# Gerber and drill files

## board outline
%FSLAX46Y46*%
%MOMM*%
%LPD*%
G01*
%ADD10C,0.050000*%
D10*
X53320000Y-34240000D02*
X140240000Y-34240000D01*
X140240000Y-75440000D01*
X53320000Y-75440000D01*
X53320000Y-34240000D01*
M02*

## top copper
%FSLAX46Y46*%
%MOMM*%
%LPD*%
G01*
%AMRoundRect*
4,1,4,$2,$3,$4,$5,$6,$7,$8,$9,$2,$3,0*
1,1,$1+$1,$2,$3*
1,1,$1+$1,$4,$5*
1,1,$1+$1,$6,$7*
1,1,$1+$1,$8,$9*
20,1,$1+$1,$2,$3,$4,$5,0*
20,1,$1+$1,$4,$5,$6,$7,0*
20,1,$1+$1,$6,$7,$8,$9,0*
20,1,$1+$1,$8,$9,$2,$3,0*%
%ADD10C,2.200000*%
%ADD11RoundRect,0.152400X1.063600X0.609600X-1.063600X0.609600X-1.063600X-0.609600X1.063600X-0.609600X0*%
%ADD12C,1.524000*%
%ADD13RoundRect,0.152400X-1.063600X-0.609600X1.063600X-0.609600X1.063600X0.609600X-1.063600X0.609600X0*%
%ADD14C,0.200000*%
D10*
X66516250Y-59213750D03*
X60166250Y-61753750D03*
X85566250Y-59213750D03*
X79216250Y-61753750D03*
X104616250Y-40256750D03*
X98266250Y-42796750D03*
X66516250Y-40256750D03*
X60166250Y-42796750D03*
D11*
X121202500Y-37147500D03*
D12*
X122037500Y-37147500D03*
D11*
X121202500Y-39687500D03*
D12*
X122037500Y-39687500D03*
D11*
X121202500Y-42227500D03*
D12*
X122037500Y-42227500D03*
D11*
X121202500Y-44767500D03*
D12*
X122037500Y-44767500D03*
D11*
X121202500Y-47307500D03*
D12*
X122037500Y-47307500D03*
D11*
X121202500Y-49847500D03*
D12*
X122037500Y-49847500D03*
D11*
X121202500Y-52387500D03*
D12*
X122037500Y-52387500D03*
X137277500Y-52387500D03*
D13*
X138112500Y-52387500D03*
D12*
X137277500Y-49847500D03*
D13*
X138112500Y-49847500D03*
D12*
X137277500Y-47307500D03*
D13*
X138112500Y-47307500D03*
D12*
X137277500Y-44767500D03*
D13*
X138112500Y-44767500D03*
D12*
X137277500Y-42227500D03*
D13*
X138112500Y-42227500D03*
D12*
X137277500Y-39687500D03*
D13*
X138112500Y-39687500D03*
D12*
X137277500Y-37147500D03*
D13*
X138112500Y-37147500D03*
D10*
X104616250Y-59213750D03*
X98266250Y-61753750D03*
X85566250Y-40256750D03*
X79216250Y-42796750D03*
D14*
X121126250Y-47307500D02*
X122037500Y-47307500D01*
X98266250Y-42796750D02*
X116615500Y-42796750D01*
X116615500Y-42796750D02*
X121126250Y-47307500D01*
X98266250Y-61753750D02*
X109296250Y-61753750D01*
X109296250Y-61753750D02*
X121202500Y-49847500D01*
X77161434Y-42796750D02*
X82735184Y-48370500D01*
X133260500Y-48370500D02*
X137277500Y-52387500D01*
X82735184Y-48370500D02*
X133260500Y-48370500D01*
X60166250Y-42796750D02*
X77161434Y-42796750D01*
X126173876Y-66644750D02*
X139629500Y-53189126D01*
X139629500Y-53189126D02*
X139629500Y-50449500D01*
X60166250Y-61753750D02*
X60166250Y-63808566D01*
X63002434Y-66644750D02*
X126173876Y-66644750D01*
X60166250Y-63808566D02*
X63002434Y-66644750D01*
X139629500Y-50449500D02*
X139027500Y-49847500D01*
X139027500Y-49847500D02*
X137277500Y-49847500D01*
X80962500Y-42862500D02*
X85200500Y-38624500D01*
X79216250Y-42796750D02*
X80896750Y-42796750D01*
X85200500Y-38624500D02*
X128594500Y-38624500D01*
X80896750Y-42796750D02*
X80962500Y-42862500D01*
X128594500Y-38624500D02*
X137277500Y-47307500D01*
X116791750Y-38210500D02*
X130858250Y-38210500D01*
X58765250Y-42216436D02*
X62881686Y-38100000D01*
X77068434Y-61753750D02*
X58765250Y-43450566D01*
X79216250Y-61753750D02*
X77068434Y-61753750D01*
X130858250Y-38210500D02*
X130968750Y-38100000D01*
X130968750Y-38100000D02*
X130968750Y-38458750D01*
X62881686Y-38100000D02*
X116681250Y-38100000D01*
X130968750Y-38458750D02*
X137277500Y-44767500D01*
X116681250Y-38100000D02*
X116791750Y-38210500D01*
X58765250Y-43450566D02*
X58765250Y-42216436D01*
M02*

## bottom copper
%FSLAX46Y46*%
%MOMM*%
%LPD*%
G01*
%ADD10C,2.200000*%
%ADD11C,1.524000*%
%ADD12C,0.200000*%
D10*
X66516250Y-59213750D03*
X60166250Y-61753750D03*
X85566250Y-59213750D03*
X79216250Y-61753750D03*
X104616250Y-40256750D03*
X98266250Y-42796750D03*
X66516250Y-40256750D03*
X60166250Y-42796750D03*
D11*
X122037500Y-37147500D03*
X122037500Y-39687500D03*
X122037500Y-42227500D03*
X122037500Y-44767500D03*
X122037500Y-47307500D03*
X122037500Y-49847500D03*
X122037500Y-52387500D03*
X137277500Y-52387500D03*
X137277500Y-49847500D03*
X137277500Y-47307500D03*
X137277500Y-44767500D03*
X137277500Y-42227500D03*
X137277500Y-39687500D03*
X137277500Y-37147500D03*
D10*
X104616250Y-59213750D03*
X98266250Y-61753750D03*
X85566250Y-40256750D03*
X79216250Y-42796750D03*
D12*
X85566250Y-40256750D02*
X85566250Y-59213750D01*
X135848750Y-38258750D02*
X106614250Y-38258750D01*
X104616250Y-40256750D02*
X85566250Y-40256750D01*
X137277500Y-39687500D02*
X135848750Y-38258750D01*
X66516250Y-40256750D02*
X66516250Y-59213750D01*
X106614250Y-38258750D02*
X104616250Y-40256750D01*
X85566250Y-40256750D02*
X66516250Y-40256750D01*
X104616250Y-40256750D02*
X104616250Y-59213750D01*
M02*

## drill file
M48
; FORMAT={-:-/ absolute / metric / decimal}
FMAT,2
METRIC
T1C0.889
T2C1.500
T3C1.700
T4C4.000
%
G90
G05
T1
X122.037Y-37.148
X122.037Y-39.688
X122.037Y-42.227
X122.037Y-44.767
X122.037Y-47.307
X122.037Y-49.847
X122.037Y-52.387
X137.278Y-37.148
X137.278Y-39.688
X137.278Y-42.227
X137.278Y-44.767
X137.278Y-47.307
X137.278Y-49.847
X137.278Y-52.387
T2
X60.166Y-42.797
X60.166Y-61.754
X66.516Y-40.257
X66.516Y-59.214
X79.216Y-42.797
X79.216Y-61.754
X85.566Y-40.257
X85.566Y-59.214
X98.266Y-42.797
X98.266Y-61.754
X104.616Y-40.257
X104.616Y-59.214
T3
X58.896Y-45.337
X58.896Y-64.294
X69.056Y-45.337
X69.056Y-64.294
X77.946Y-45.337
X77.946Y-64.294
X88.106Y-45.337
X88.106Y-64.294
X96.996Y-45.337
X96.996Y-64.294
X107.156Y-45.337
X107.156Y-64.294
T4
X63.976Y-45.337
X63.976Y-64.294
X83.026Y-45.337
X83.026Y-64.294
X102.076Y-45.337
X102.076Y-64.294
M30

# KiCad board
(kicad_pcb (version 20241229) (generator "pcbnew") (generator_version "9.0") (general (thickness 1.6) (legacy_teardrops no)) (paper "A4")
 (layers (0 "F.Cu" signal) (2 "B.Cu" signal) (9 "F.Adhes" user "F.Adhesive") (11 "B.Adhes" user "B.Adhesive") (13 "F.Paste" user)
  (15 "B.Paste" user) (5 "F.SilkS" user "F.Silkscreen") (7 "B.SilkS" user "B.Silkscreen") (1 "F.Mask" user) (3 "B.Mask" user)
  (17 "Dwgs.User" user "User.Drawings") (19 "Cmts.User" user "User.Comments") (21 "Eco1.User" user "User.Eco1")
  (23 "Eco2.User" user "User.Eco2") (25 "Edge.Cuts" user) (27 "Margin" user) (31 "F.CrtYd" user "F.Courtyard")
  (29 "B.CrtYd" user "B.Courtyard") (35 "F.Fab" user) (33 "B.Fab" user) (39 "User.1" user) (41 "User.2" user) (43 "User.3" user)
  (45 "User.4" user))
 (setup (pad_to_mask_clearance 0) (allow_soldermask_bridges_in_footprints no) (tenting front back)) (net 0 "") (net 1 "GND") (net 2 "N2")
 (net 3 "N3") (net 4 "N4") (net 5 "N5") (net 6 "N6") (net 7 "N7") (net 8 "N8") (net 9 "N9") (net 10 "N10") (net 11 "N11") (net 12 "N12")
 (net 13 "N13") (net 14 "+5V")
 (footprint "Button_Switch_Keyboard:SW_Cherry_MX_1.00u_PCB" (layer "F.Cu") (at 66.51625 59.21375)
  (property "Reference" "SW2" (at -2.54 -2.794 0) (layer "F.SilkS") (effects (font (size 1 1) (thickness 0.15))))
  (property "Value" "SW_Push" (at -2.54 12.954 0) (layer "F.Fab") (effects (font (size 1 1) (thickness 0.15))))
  (pad "" np_thru_hole circle (at -7.62 5.08) (size 1.7 1.7) (drill 1.7) (layers "*.Cu" "*.Mask"))
  (pad "" np_thru_hole circle (at -2.54 5.08) (size 4 4) (drill 4) (layers "*.Cu" "*.Mask"))
  (pad "" np_thru_hole circle (at 2.54 5.08) (size 1.7 1.7) (drill 1.7) (layers "*.Cu" "*.Mask"))
  (pad "1" thru_hole circle (at 0 0) (size 2.2 2.2) (drill 1.5) (layers "*.Cu" "*.Mask") (remove_unused_layers no) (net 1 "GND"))
  (pad "2" thru_hole circle (at -6.35 2.54) (size 2.2 2.2) (drill 1.5) (layers "*.Cu" "*.Mask") (remove_unused_layers no) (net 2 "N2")))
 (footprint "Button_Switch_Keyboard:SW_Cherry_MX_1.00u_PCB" (layer "F.Cu") (at 85.56625 59.21375)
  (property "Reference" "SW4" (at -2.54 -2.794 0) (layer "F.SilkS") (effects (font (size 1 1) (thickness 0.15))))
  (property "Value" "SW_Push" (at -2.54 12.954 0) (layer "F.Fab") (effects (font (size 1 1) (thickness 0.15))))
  (pad "" np_thru_hole circle (at -7.62 5.08) (size 1.7 1.7) (drill 1.7) (layers "*.Cu" "*.Mask"))
  (pad "" np_thru_hole circle (at -2.54 5.08) (size 4 4) (drill 4) (layers "*.Cu" "*.Mask"))
  (pad "" np_thru_hole circle (at 2.54 5.08) (size 1.7 1.7) (drill 1.7) (layers "*.Cu" "*.Mask"))
  (pad "1" thru_hole circle (at 0 0) (size 2.2 2.2) (drill 1.5) (layers "*.Cu" "*.Mask") (remove_unused_layers no) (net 1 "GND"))
  (pad "2" thru_hole circle (at -6.35 2.54) (size 2.2 2.2) (drill 1.5) (layers "*.Cu" "*.Mask") (remove_unused_layers no) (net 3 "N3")))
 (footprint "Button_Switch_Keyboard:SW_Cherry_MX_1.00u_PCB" (layer "F.Cu") (at 104.61625 40.25675)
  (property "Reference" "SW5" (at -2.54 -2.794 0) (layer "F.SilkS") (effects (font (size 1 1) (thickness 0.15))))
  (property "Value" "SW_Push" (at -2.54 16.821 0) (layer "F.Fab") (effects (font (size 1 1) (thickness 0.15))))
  (pad "" np_thru_hole circle (at -7.62 5.08) (size 1.7 1.7) (drill 1.7) (layers "*.Cu" "*.Mask"))
  (pad "" np_thru_hole circle (at -2.54 5.08) (size 4 4) (drill 4) (layers "*.Cu" "*.Mask"))
  (pad "" np_thru_hole circle (at 2.54 5.08) (size 1.7 1.7) (drill 1.7) (layers "*.Cu" "*.Mask"))
  (pad "1" thru_hole circle (at 0 0) (size 2.2 2.2) (drill 1.5) (layers "*.Cu" "*.Mask") (remove_unused_layers no) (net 1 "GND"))
  (pad "2" thru_hole circle (at -6.35 2.54) (size 2.2 2.2) (drill 1.5) (layers "*.Cu" "*.Mask") (remove_unused_layers no) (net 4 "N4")))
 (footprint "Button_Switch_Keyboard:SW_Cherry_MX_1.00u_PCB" (layer "F.Cu") (at 66.51625 40.25675)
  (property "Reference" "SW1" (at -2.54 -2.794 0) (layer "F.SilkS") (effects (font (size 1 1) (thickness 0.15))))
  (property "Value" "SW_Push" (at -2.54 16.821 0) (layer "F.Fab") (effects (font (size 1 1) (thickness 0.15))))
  (pad "" np_thru_hole circle (at -7.62 5.08) (size 1.7 1.7) (drill 1.7) (layers "*.Cu" "*.Mask"))
  (pad "" np_thru_hole circle (at -2.54 5.08) (size 4 4) (drill 4) (layers "*.Cu" "*.Mask"))
  (pad "" np_thru_hole circle (at 2.54 5.08) (size 1.7 1.7) (drill 1.7) (layers "*.Cu" "*.Mask"))
  (pad "1" thru_hole circle (at 0 0) (size 2.2 2.2) (drill 1.5) (layers "*.Cu" "*.Mask") (remove_unused_layers no) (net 1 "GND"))
  (pad "2" thru_hole circle (at -6.35 2.54) (size 2.2 2.2) (drill 1.5) (layers "*.Cu" "*.Mask") (remove_unused_layers no) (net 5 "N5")))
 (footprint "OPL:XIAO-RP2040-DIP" (layer "F.Cu") (at 129.6575 44.7675)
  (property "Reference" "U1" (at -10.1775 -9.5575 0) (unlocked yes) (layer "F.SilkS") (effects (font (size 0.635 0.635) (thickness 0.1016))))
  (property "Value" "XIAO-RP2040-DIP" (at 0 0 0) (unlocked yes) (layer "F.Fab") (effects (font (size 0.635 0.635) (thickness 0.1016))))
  (pad "1" smd roundrect (at -8.455 -7.62 180) (size 2.432 1.524) (layers "F.Cu" "F.Mask") (roundrect_rratio 0.1) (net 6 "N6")
   (thermal_bridge_angle 45))
  (pad "1" thru_hole circle (at -7.62 -7.62 180) (size 1.524 1.524) (drill 0.889) (layers "*.Cu" "*.Mask") (remove_unused_layers no)
   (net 6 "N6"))
  (pad "2" smd roundrect (at -8.455 -5.08 180) (size 2.432 1.524) (layers "F.Cu" "F.Mask") (roundrect_rratio 0.1) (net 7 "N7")
   (thermal_bridge_angle 45))
  (pad "2" thru_hole circle (at -7.62 -5.08 180) (size 1.524 1.524) (drill 0.889) (layers "*.Cu" "*.Mask") (remove_unused_layers no)
   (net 7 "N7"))
  (pad "3" smd roundrect (at -8.455 -2.54 180) (size 2.432 1.524) (layers "F.Cu" "F.Mask") (roundrect_rratio 0.1) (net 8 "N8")
   (thermal_bridge_angle 45))
  (pad "3" thru_hole circle (at -7.62 -2.54 180) (size 1.524 1.524) (drill 0.889) (layers "*.Cu" "*.Mask") (remove_unused_layers no)
   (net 8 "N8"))
  (pad "4" smd roundrect (at -8.455 0 180) (size 2.432 1.524) (layers "F.Cu" "F.Mask") (roundrect_rratio 0.1) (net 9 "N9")
   (thermal_bridge_angle 45))
  (pad "4" thru_hole circle (at -7.62 0 180) (size 1.524 1.524) (drill 0.889) (layers "*.Cu" "*.Mask") (remove_unused_layers no)
   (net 9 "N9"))
  (pad "5" smd roundrect (at -8.455 2.54 180) (size 2.432 1.524) (layers "F.Cu" "F.Mask") (roundrect_rratio 0.1) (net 4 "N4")
   (thermal_bridge_angle 45))
  (pad "5" thru_hole circle (at -7.62 2.54 180) (size 1.524 1.524) (drill 0.889) (layers "*.Cu" "*.Mask") (remove_unused_layers no)
   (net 4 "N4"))
  (pad "6" smd roundrect (at -8.455 5.08 180) (size 2.432 1.524) (layers "F.Cu" "F.Mask") (roundrect_rratio 0.1) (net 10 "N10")
   (thermal_bridge_angle 45))
  (pad "6" thru_hole circle (at -7.62 5.08 180) (size 1.524 1.524) (drill 0.889) (layers "*.Cu" "*.Mask") (remove_unused_layers no)
   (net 10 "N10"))
  (pad "7" smd roundrect (at -8.455 7.62 180) (size 2.432 1.524) (layers "F.Cu" "F.Mask") (roundrect_rratio 0.1) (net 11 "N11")
   (thermal_bridge_angle 45))
  (pad "7" thru_hole circle (at -7.62 7.62 180) (size 1.524 1.524) (drill 0.889) (layers "*.Cu" "*.Mask") (remove_unused_layers no)
   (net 11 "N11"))
  (pad "8" thru_hole circle (at 7.62 7.62) (size 1.524 1.524) (drill 0.889) (layers "*.Cu" "*.Mask") (remove_unused_layers no) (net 5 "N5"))
  (pad "8" smd roundrect (at 8.455 7.62) (size 2.432 1.524) (layers "F.Cu" "F.Mask") (roundrect_rratio 0.1) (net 5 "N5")
   (thermal_bridge_angle 45))
  (pad "9" thru_hole circle (at 7.62 5.08) (size 1.524 1.524) (drill 0.889) (layers "*.Cu" "*.Mask") (remove_unused_layers no) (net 2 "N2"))
  (pad "9" smd roundrect (at 8.455 5.08) (size 2.432 1.524) (layers "F.Cu" "F.Mask") (roundrect_rratio 0.1) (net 2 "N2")
   (thermal_bridge_angle 45))
  (pad "10" thru_hole circle (at 7.62 2.54) (size 1.524 1.524) (drill 0.889) (layers "*.Cu" "*.Mask") (remove_unused_layers no)
   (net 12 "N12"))
  (pad "10" smd roundrect (at 8.455 2.54) (size 2.432 1.524) (layers "F.Cu" "F.Mask") (roundrect_rratio 0.1) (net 12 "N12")
   (thermal_bridge_angle 45))
  (pad "11" thru_hole circle (at 7.62 0) (size 1.524 1.524) (drill 0.889) (layers "*.Cu" "*.Mask") (remove_unused_layers no) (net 3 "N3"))
  (pad "11" smd roundrect (at 8.455 0) (size 2.432 1.524) (layers "F.Cu" "F.Mask") (roundrect_rratio 0.1) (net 3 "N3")
   (thermal_bridge_angle 45))
  (pad "12" thru_hole circle (at 7.62 -2.54) (size 1.524 1.524) (drill 0.889) (layers "*.Cu" "*.Mask") (remove_unused_layers no)
   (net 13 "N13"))
  (pad "12" smd roundrect (at 8.455 -2.54) (size 2.432 1.524) (layers "F.Cu" "F.Mask") (roundrect_rratio 0.1) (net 13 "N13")
   (thermal_bridge_angle 45))
  (pad "13" thru_hole circle (at 7.62 -5.08) (size 1.524 1.524) (drill 0.889) (layers "*.Cu" "*.Mask") (remove_unused_layers no)
   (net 1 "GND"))
  (pad "13" smd roundrect (at 8.455 -5.08) (size 2.432 1.524) (layers "F.Cu" "F.Mask") (roundrect_rratio 0.1) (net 1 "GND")
   (thermal_bridge_angle 45))
  (pad "14" thru_hole circle (at 7.62 -7.62) (size 1.524 1.524) (drill 0.889) (layers "*.Cu" "*.Mask") (remove_unused_layers no)
   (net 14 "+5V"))
  (pad "14" smd roundrect (at 8.455 -7.62) (size 2.432 1.524) (layers "F.Cu" "F.Mask") (roundrect_rratio 0.1) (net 14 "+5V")
   (thermal_bridge_angle 45)))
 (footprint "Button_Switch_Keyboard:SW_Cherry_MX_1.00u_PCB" (layer "F.Cu") (at 104.61625 59.21375)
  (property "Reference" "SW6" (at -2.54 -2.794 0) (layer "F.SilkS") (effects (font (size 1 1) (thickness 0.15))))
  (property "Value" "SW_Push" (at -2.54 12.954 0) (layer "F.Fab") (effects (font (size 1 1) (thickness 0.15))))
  (pad "" np_thru_hole circle (at -7.62 5.08) (size 1.7 1.7) (drill 1.7) (layers "*.Cu" "*.Mask"))
  (pad "" np_thru_hole circle (at -2.54 5.08) (size 4 4) (drill 4) (layers "*.Cu" "*.Mask"))
  (pad "" np_thru_hole circle (at 2.54 5.08) (size 1.7 1.7) (drill 1.7) (layers "*.Cu" "*.Mask"))
  (pad "1" thru_hole circle (at 0 0) (size 2.2 2.2) (drill 1.5) (layers "*.Cu" "*.Mask") (remove_unused_layers no) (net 1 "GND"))
  (pad "2" thru_hole circle (at -6.35 2.54) (size 2.2 2.2) (drill 1.5) (layers "*.Cu" "*.Mask") (remove_unused_layers no) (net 10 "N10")))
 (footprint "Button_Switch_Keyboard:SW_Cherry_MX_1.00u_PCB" (layer "F.Cu") (at 85.56625 40.25675)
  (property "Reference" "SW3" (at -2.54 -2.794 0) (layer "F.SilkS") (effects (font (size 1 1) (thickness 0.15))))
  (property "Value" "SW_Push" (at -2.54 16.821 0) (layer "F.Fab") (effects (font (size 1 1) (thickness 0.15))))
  (pad "" np_thru_hole circle (at -7.62 5.08) (size 1.7 1.7) (drill 1.7) (layers "*.Cu" "*.Mask"))
  (pad "" np_thru_hole circle (at -2.54 5.08) (size 4 4) (drill 4) (layers "*.Cu" "*.Mask"))
  (pad "" np_thru_hole circle (at 2.54 5.08) (size 1.7 1.7) (drill 1.7) (layers "*.Cu" "*.Mask"))
  (pad "1" thru_hole circle (at 0 0) (size 2.2 2.2) (drill 1.5) (layers "*.Cu" "*.Mask") (remove_unused_layers no) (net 1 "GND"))
  (pad "2" thru_hole circle (at -6.35 2.54) (size 2.2 2.2) (drill 1.5) (layers "*.Cu" "*.Mask") (remove_unused_layers no) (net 12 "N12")))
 (gr_rect (start 53.32 34.24) (end 140.24 75.44) (stroke (width 0.05) (type default)) (fill no) (layer "Edge.Cuts"))
 (segment (start 121.12625 47.3075) (end 122.0375 47.3075) (width 0.2) (layer "F.Cu") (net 4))
 (segment (start 98.26625 42.79675) (end 116.6155 42.79675) (width 0.2) (layer "F.Cu") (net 4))
 (segment (start 116.6155 42.79675) (end 121.12625 47.3075) (width 0.2) (layer "F.Cu") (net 4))
 (segment (start 85.56625 40.25675) (end 85.56625 59.21375) (width 0.2) (layer "B.Cu") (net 1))
 (segment (start 135.84875 38.25875) (end 106.61425 38.25875) (width 0.2) (layer "B.Cu") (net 1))
 (segment (start 104.61625 40.25675) (end 85.56625 40.25675) (width 0.2) (layer "B.Cu") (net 1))
 (segment (start 137.2775 39.6875) (end 135.84875 38.25875) (width 0.2) (layer "B.Cu") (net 1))
 (segment (start 66.51625 40.25675) (end 66.51625 59.21375) (width 0.2) (layer "B.Cu") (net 1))
 (segment (start 106.61425 38.25875) (end 104.61625 40.25675) (width 0.2) (layer "B.Cu") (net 1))
 (segment (start 85.56625 40.25675) (end 66.51625 40.25675) (width 0.2) (layer "B.Cu") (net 1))
 (segment (start 104.61625 40.25675) (end 104.61625 59.21375) (width 0.2) (layer "B.Cu") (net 1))
 (segment (start 98.26625 61.75375) (end 109.29625 61.75375) (width 0.2) (layer "F.Cu") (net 10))
 (segment (start 109.29625 61.75375) (end 121.2025 49.8475) (width 0.2) (layer "F.Cu") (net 10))
 (segment (start 77.161434 42.79675) (end 82.735184 48.3705) (width 0.2) (layer "F.Cu") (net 5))
 (segment (start 133.2605 48.3705) (end 137.2775 52.3875) (width 0.2) (layer "F.Cu") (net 5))
 (segment (start 82.735184 48.3705) (end 133.2605 48.3705) (width 0.2) (layer "F.Cu") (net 5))
 (segment (start 60.16625 42.79675) (end 77.161434 42.79675) (width 0.2) (layer "F.Cu") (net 5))
 (segment (start 126.173876 66.64475) (end 139.6295 53.189126) (width 0.2) (layer "F.Cu") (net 2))
 (segment (start 139.6295 53.189126) (end 139.6295 50.4495) (width 0.2) (layer "F.Cu") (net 2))
 (segment (start 60.16625 61.75375) (end 60.16625 63.808566) (width 0.2) (layer "F.Cu") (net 2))
 (segment (start 63.002434 66.64475) (end 126.173876 66.64475) (width 0.2) (layer "F.Cu") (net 2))
 (segment (start 60.16625 63.808566) (end 63.002434 66.64475) (width 0.2) (layer "F.Cu") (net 2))
 (segment (start 139.6295 50.4495) (end 139.0275 49.8475) (width 0.2) (layer "F.Cu") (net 2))
 (segment (start 139.0275 49.8475) (end 137.2775 49.8475) (width 0.2) (layer "F.Cu") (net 2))
 (segment (start 80.9625 42.8625) (end 85.2005 38.6245) (width 0.2) (layer "F.Cu") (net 12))
 (segment (start 79.21625 42.79675) (end 80.89675 42.79675) (width 0.2) (layer "F.Cu") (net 12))
 (segment (start 85.2005 38.6245) (end 128.5945 38.6245) (width 0.2) (layer "F.Cu") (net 12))
 (segment (start 80.89675 42.79675) (end 80.9625 42.8625) (width 0.2) (layer "F.Cu") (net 12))
 (segment (start 128.5945 38.6245) (end 137.2775 47.3075) (width 0.2) (layer "F.Cu") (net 12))
 (segment (start 116.79175 38.2105) (end 130.85825 38.2105) (width 0.2) (layer "F.Cu") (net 3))
 (segment (start 58.76525 42.216436) (end 62.881686 38.1) (width 0.2) (layer "F.Cu") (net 3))
 (segment (start 77.068434 61.75375) (end 58.76525 43.450566) (width 0.2) (layer "F.Cu") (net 3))
 (segment (start 79.21625 61.75375) (end 77.068434 61.75375) (width 0.2) (layer "F.Cu") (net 3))
 (segment (start 130.85825 38.2105) (end 130.96875 38.1) (width 0.2) (layer "F.Cu") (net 3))
 (segment (start 130.96875 38.1) (end 130.96875 38.45875) (width 0.2) (layer "F.Cu") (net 3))
 (segment (start 62.881686 38.1) (end 116.68125 38.1) (width 0.2) (layer "F.Cu") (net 3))
 (segment (start 130.96875 38.45875) (end 137.2775 44.7675) (width 0.2) (layer "F.Cu") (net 3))
 (segment (start 116.68125 38.1) (end 116.79175 38.2105) (width 0.2) (layer "F.Cu") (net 3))
 (segment (start 58.76525 43.450566) (end 58.76525 42.216436) (width 0.2) (layer "F.Cu") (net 3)))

